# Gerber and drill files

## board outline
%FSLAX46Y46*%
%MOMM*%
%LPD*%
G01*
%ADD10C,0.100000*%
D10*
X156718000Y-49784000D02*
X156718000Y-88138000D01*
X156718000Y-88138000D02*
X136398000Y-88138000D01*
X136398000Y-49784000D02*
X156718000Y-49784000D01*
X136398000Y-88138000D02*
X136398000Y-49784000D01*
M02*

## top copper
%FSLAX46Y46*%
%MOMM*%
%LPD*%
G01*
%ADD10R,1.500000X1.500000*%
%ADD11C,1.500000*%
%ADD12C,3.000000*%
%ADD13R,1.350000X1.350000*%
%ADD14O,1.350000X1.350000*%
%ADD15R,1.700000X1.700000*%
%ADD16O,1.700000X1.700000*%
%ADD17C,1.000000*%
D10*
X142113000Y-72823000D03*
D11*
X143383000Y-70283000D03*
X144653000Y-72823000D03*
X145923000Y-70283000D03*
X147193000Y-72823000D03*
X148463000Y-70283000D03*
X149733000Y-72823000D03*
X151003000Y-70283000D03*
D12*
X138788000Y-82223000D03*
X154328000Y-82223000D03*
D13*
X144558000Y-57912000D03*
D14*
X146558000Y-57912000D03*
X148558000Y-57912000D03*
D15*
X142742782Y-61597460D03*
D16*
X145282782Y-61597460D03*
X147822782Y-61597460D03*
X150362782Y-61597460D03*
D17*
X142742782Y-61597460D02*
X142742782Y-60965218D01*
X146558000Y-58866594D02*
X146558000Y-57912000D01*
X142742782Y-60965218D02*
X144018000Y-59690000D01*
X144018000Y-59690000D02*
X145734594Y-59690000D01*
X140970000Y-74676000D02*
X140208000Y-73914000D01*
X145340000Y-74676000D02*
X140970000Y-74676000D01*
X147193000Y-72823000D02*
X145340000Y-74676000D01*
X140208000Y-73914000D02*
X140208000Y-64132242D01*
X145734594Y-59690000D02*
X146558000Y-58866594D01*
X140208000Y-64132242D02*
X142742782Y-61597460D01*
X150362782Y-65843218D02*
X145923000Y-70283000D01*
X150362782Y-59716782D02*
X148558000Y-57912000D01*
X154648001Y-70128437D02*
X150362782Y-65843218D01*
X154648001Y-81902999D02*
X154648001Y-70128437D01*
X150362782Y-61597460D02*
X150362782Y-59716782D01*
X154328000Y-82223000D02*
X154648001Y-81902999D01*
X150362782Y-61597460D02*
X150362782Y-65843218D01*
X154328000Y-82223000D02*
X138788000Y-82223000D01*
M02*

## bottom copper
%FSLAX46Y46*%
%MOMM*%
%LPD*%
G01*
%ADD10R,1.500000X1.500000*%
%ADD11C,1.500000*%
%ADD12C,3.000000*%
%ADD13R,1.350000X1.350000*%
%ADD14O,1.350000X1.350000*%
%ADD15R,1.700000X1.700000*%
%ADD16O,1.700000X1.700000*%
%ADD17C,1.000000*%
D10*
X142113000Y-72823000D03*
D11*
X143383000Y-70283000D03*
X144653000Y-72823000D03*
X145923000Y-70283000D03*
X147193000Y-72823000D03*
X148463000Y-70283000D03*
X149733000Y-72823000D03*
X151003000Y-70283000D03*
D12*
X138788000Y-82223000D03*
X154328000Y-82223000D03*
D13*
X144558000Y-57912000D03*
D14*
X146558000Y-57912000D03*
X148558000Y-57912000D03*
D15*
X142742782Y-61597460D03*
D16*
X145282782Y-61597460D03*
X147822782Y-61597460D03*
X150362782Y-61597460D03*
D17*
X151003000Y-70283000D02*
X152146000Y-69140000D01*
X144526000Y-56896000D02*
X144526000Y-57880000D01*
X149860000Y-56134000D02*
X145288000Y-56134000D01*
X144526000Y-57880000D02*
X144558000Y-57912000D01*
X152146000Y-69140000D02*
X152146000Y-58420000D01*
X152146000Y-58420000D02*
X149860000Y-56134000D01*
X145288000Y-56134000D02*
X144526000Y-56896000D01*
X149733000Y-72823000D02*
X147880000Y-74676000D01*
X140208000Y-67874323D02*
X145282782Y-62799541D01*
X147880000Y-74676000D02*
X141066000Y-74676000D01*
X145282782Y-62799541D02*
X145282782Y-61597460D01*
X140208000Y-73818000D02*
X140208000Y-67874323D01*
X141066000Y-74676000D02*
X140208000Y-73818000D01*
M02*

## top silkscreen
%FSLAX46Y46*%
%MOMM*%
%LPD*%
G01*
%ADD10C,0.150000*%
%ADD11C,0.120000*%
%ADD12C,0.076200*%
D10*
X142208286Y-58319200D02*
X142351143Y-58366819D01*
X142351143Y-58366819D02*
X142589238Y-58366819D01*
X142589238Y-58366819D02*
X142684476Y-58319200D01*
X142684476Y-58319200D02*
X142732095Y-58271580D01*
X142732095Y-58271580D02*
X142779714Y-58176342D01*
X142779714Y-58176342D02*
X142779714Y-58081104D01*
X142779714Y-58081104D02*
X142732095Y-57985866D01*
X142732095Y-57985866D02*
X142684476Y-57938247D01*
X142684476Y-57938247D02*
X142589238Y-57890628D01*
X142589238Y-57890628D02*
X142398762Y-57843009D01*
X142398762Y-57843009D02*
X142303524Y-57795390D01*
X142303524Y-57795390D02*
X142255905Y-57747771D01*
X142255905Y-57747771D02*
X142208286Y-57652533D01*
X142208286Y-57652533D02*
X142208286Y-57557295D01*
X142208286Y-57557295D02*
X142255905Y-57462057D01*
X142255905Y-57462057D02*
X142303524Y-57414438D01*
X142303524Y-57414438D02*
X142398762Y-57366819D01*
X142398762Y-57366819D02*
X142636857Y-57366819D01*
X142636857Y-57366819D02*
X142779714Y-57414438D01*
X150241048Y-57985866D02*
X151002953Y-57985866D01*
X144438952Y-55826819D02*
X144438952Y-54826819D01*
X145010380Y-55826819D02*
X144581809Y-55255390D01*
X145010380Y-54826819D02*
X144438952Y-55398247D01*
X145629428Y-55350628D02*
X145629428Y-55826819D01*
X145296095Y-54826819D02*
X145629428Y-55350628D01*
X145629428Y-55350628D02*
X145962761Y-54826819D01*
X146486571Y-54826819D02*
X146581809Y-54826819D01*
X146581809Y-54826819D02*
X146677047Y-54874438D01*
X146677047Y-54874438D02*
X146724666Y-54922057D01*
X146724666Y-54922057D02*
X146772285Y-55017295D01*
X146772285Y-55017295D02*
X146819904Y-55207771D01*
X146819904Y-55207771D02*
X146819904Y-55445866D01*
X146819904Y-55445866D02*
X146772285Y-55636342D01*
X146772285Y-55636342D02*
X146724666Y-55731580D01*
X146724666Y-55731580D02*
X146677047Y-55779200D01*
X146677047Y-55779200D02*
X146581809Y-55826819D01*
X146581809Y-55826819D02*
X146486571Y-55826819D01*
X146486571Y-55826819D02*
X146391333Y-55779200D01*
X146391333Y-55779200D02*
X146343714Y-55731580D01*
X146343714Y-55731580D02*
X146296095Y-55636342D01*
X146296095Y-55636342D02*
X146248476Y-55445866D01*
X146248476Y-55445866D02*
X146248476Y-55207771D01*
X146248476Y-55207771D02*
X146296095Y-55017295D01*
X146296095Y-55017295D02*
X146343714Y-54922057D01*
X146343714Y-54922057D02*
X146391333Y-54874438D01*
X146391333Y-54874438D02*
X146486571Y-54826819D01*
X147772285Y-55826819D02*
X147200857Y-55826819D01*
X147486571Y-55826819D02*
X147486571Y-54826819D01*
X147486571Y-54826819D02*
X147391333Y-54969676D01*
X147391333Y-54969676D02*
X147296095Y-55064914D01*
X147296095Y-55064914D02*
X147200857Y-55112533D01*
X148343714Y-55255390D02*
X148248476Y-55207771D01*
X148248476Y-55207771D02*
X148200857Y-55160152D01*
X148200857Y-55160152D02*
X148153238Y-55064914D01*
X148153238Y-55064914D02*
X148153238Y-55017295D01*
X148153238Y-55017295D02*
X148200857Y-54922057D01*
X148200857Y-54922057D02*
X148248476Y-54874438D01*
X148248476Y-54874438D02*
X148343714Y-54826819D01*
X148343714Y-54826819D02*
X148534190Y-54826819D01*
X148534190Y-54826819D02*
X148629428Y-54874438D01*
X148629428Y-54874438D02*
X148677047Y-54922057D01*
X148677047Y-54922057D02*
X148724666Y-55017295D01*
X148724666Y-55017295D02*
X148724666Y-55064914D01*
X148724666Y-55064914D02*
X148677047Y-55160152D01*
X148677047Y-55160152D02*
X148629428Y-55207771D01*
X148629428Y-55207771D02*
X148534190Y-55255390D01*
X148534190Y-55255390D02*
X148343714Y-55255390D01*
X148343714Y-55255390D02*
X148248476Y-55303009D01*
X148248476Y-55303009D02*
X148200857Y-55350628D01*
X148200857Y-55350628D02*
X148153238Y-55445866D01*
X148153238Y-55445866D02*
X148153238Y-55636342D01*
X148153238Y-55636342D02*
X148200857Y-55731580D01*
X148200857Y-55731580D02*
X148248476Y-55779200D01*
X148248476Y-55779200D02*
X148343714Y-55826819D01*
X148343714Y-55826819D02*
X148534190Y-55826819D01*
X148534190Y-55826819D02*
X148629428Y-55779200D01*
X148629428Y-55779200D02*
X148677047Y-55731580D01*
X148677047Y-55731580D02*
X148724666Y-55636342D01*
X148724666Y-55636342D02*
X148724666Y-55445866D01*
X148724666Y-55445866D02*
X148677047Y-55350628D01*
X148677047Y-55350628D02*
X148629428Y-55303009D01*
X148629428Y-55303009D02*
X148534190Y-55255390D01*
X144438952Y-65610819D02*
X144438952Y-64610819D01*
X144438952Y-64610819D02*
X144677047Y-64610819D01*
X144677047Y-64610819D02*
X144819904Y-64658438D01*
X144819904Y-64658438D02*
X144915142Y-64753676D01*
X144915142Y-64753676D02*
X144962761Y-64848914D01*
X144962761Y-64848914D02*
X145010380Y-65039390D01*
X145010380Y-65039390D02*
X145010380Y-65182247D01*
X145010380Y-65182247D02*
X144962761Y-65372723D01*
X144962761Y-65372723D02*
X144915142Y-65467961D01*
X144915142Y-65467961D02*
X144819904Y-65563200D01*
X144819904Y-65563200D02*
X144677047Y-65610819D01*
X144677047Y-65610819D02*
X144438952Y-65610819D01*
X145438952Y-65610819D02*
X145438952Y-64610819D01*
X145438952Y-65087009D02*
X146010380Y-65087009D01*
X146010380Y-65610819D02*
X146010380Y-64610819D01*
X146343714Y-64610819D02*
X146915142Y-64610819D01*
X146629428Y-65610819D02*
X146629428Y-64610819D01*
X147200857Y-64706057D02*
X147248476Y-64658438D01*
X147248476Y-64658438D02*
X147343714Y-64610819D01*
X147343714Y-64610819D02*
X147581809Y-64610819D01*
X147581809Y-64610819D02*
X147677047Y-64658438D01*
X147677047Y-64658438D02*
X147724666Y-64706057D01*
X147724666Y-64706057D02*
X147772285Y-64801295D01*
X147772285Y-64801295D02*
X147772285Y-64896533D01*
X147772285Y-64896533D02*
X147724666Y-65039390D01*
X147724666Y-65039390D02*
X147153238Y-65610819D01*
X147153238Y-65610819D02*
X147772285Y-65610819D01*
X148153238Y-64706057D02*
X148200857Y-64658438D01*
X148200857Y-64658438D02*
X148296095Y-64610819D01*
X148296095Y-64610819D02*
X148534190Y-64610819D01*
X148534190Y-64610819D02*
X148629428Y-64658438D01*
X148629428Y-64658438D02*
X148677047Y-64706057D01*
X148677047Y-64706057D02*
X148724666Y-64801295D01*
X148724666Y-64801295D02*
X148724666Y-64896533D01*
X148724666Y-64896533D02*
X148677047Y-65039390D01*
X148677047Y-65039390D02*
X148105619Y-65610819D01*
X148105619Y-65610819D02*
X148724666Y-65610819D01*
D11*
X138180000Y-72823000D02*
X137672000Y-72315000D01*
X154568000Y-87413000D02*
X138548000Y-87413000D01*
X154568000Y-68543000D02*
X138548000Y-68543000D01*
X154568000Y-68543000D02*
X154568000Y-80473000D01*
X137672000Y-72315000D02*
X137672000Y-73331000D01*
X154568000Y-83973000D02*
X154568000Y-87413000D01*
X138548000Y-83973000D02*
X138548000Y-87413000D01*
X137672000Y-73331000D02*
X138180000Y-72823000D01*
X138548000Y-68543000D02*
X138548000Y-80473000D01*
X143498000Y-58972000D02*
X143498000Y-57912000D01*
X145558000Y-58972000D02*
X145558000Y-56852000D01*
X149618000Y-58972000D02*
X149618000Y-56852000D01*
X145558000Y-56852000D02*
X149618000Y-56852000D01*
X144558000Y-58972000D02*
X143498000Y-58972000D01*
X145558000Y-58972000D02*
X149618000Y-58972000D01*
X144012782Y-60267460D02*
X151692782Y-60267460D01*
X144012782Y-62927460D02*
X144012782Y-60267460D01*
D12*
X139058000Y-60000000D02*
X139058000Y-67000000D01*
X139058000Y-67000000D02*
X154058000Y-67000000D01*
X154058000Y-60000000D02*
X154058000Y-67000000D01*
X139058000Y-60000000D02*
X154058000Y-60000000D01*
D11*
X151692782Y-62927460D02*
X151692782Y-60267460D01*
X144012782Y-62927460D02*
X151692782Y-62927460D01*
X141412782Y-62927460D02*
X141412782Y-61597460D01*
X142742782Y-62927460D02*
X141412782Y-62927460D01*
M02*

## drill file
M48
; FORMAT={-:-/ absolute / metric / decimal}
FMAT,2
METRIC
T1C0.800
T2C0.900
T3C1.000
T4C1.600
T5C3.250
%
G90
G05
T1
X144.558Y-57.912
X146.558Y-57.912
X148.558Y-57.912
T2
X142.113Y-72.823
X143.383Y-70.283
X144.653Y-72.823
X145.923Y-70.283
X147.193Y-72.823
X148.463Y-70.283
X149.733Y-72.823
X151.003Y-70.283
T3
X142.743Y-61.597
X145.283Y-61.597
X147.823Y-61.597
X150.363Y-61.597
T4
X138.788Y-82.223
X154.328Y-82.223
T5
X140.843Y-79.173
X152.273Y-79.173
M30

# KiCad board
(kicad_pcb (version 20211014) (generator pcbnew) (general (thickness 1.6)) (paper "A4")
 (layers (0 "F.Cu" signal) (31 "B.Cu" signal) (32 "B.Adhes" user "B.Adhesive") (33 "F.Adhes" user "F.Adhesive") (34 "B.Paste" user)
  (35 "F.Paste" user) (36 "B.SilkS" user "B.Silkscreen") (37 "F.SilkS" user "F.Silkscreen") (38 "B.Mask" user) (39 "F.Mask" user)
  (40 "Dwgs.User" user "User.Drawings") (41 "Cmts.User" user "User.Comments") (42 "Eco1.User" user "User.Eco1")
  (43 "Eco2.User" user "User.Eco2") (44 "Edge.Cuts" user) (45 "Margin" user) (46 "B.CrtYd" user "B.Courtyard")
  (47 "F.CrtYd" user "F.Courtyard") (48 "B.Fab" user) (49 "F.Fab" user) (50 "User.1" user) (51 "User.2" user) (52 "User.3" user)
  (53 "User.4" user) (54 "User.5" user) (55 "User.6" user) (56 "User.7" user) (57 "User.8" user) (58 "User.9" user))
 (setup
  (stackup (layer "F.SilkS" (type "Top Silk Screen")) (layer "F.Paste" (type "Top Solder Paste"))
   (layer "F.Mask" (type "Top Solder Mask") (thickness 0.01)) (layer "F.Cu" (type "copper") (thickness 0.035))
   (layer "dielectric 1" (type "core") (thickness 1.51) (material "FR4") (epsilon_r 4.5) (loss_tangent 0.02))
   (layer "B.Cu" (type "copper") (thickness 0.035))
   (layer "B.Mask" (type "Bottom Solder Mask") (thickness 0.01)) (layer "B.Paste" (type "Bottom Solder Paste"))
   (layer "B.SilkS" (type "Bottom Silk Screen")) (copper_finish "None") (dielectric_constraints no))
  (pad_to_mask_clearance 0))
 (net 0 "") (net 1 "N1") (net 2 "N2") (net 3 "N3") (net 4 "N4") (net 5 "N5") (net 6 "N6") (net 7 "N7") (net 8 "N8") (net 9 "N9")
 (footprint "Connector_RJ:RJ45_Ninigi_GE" (layer "F.Cu") (at 142.113 72.823)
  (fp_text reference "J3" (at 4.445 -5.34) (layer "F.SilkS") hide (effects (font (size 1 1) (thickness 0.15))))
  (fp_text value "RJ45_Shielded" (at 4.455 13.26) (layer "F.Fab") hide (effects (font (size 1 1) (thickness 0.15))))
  (fp_line (start -3.933 0) (end -4.441 -0.508) (layer "F.SilkS") (width 0.12))
  (fp_line (start 12.455 14.59) (end -3.565 14.59) (layer "F.SilkS") (width 0.12))
  (fp_line (start 12.455 -4.28) (end -3.565 -4.28) (layer "F.SilkS") (width 0.12))
  (fp_line (start 12.455 -4.28) (end 12.455 7.65) (layer "F.SilkS") (width 0.12))
  (fp_line (start -4.441 -0.508) (end -4.441 0.508) (layer "F.SilkS") (width 0.12))
  (fp_line (start 12.455 11.15) (end 12.455 14.59) (layer "F.SilkS") (width 0.12))
  (fp_line (start -3.565 11.15) (end -3.565 14.59) (layer "F.SilkS") (width 0.12))
  (fp_line (start -4.441 0.508) (end -3.933 0) (layer "F.SilkS") (width 0.12))
  (fp_line (start -3.565 -4.28) (end -3.565 7.65) (layer "F.SilkS") (width 0.12))
  (pad "" np_thru_hole circle (at -1.27 6.35) (size 3.25 3.25) (drill 3.25) (layers *.Cu *.Mask))
  (pad "" np_thru_hole circle (at 10.16 6.35 180) (size 3.25 3.25) (drill 3.25) (layers *.Cu *.Mask))
  (pad "1" thru_hole rect (at 0 0 180) (size 1.5 1.5) (drill 0.9) (layers *.Cu *.Mask) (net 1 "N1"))
  (pad "2" thru_hole circle (at 1.27 -2.54 180) (size 1.5 1.5) (drill 0.9) (layers *.Cu *.Mask) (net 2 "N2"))
  (pad "3" thru_hole circle (at 2.54 0 180) (size 1.5 1.5) (drill 0.9) (layers *.Cu *.Mask) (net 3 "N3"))
  (pad "4" thru_hole circle (at 3.81 -2.54 180) (size 1.5 1.5) (drill 0.9) (layers *.Cu *.Mask) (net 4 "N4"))
  (pad "5" thru_hole circle (at 5.08 0 180) (size 1.5 1.5) (drill 0.9) (layers *.Cu *.Mask) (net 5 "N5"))
  (pad "6" thru_hole circle (at 6.35 -2.54 180) (size 1.5 1.5) (drill 0.9) (layers *.Cu *.Mask) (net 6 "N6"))
  (pad "7" thru_hole circle (at 7.62 0 180) (size 1.5 1.5) (drill 0.9) (layers *.Cu *.Mask) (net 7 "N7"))
  (pad "8" thru_hole circle (at 8.89 -2.54 180) (size 1.5 1.5) (drill 0.9) (layers *.Cu *.Mask) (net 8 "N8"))
  (pad "SH" thru_hole circle (at -3.325 9.4) (size 3 3) (drill 1.6) (layers *.Cu *.Mask) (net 4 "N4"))
  (pad "SH" thru_hole circle (at 12.215 9.4 180) (size 3 3) (drill 1.6) (layers *.Cu *.Mask) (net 4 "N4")))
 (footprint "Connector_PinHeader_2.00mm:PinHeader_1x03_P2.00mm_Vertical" (layer "F.Cu") (at 144.558 57.912 90)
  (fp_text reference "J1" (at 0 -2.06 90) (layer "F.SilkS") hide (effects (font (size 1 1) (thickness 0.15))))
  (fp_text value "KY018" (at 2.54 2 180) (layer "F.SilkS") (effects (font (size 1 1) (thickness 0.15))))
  (fp_line (start -1.06 -1.06) (end 0 -1.06) (layer "F.SilkS") (width 0.12))
  (fp_line (start -1.06 1) (end 1.06 1) (layer "F.SilkS") (width 0.12))
  (fp_line (start -1.06 5.06) (end 1.06 5.06) (layer "F.SilkS") (width 0.12))
  (fp_line (start 1.06 1) (end 1.06 5.06) (layer "F.SilkS") (width 0.12))
  (fp_line (start -1.06 0) (end -1.06 -1.06) (layer "F.SilkS") (width 0.12))
  (fp_line (start -1.06 1) (end -1.06 5.06) (layer "F.SilkS") (width 0.12))
  (pad "1" thru_hole rect (at 0 0 90) (size 1.35 1.35) (drill 0.8) (layers *.Cu *.Mask) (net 8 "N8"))
  (pad "2" thru_hole oval (at 0 2 90) (size 1.35 1.35) (drill 0.8) (layers *.Cu *.Mask) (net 5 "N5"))
  (pad "3" thru_hole oval (at 0 4 90) (size 1.35 1.35) (drill 0.8) (layers *.Cu *.Mask) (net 4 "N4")))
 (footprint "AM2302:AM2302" (layer "F.Cu") (at 146.558 61.6)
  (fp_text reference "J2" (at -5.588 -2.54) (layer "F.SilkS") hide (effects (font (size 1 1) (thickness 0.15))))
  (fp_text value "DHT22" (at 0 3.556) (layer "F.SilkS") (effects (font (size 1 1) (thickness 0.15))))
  (fp_line (start -2.545218 -1.33254) (end 5.134782 -1.33254) (layer "F.SilkS") (width 0.12))
  (fp_line (start -2.545218 1.32746) (end -2.545218 -1.33254) (layer "F.SilkS") (width 0.12))
  (fp_line (start -7.5 -1.6) (end -7.5 5.4) (layer "F.SilkS") (width 0.0762))
  (fp_line (start -7.5 5.4) (end 7.5 5.4) (layer "F.SilkS") (width 0.0762))
  (fp_line (start 7.5 -1.6) (end 7.5 5.4) (layer "F.SilkS") (width 0.0762))
  (fp_line (start -7.5 -1.6) (end 7.5 -1.6) (layer "F.SilkS") (width 0.0762))
  (fp_line (start 5.134782 1.32746) (end 5.134782 -1.33254) (layer "F.SilkS") (width 0.12))
  (fp_line (start -2.545218 1.32746) (end 5.134782 1.32746) (layer "F.SilkS") (width 0.12))
  (fp_line (start -5.145218 1.32746) (end -5.145218 -0.00254) (layer "F.SilkS") (width 0.12))
  (fp_line (start -3.815218 1.32746) (end -5.145218 1.32746) (layer "F.SilkS") (width 0.12))
  (pad "1" thru_hole rect locked (at -3.815218 -0.00254 270) (size 1.7 1.7) (drill 1) (layers *.Cu *.Mask) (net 5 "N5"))
  (pad "2" thru_hole oval locked (at -1.275218 -0.00254 90) (size 1.7 1.7) (drill 1) (layers *.Cu *.Mask) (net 7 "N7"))
  (pad "3" thru_hole oval locked (at 1.264782 -0.00254 90) (size 1.7 1.7) (drill 1) (layers *.Cu *.Mask) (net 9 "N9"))
  (pad "4" thru_hole oval locked (at 3.804782 -0.00254 90) (size 1.7 1.7) (drill 1) (layers *.Cu *.Mask) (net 4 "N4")))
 (gr_line (start 156.718 49.784) (end 156.718 88.138) (layer "Edge.Cuts") (width 0.1))
 (gr_line (start 156.718 88.138) (end 136.398 88.138) (layer "Edge.Cuts") (width 0.1))
 (gr_line (start 136.398 49.784) (end 156.718 49.784) (layer "Edge.Cuts") (width 0.1))
 (gr_line (start 136.398 88.138) (end 136.398 49.784) (layer "Edge.Cuts") (width 0.1))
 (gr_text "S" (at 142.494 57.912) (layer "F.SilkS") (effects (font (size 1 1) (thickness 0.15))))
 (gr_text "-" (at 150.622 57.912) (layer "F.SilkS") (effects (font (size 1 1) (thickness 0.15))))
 (segment (start 151.003 70.283) (end 152.146 69.14) (width 1) (layer "B.Cu") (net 8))
 (segment (start 144.526 56.896) (end 144.526 57.88) (width 1) (layer "B.Cu") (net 8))
 (segment (start 149.86 56.134) (end 145.288 56.134) (width 1) (layer "B.Cu") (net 8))
 (segment (start 144.526 57.88) (end 144.558 57.912) (width 1) (layer "B.Cu") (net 8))
 (segment (start 152.146 69.14) (end 152.146 58.42) (width 1) (layer "B.Cu") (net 8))
 (segment (start 152.146 58.42) (end 149.86 56.134) (width 1) (layer "B.Cu") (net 8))
 (segment (start 145.288 56.134) (end 144.526 56.896) (width 1) (layer "B.Cu") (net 8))
 (segment (start 142.742782 61.59746) (end 142.742782 60.965218) (width 1) (layer "F.Cu") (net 5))
 (segment (start 146.558 58.866594) (end 146.558 57.912) (width 1) (layer "F.Cu") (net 5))
 (segment (start 142.742782 60.965218) (end 144.018 59.69) (width 1) (layer "F.Cu") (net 5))
 (segment (start 144.018 59.69) (end 145.734594 59.69) (width 1) (layer "F.Cu") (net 5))
 (segment (start 140.97 74.676) (end 140.208 73.914) (width 1) (layer "F.Cu") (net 5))
 (segment (start 145.34 74.676) (end 140.97 74.676) (width 1) (layer "F.Cu") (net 5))
 (segment (start 147.193 72.823) (end 145.34 74.676) (width 1) (layer "F.Cu") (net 5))
 (segment (start 140.208 73.914) (end 140.208 64.132242) (width 1) (layer "F.Cu") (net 5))
 (segment (start 145.734594 59.69) (end 146.558 58.866594) (width 1) (layer "F.Cu") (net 5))
 (segment (start 140.208 64.132242) (end 142.742782 61.59746) (width 1) (layer "F.Cu") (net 5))
 (segment (start 150.362782 65.843218) (end 145.923 70.283) (width 1) (layer "F.Cu") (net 4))
 (segment (start 150.362782 59.716782) (end 148.558 57.912) (width 1) (layer "F.Cu") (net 4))
 (segment (start 154.648001 70.128437) (end 150.362782 65.843218) (width 1) (layer "F.Cu") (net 4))
 (segment (start 154.648001 81.902999) (end 154.648001 70.128437) (width 1) (layer "F.Cu") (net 4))
 (segment (start 150.362782 61.59746) (end 150.362782 59.716782) (width 1) (layer "F.Cu") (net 4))
 (segment (start 154.328 82.223) (end 154.648001 81.902999) (width 1) (layer "F.Cu") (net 4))
 (segment (start 150.362782 61.59746) (end 150.362782 65.843218) (width 1) (layer "F.Cu") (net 4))
 (segment (start 154.328 82.223) (end 138.788 82.223) (width 1) (layer "F.Cu") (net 4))
 (segment (start 149.733 72.823) (end 147.88 74.676) (width 1) (layer "B.Cu") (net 7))
 (segment (start 140.208 67.874323) (end 145.282782 62.799541) (width 1) (layer "B.Cu") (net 7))
 (segment (start 147.88 74.676) (end 141.066 74.676) (width 1) (layer "B.Cu") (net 7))
 (segment (start 145.282782 62.799541) (end 145.282782 61.59746) (width 1) (layer "B.Cu") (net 7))
 (segment (start 140.208 73.818) (end 140.208 67.874323) (width 1) (layer "B.Cu") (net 7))
 (segment (start 141.066 74.676) (end 140.208 73.818) (width 1) (layer "B.Cu") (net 7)))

